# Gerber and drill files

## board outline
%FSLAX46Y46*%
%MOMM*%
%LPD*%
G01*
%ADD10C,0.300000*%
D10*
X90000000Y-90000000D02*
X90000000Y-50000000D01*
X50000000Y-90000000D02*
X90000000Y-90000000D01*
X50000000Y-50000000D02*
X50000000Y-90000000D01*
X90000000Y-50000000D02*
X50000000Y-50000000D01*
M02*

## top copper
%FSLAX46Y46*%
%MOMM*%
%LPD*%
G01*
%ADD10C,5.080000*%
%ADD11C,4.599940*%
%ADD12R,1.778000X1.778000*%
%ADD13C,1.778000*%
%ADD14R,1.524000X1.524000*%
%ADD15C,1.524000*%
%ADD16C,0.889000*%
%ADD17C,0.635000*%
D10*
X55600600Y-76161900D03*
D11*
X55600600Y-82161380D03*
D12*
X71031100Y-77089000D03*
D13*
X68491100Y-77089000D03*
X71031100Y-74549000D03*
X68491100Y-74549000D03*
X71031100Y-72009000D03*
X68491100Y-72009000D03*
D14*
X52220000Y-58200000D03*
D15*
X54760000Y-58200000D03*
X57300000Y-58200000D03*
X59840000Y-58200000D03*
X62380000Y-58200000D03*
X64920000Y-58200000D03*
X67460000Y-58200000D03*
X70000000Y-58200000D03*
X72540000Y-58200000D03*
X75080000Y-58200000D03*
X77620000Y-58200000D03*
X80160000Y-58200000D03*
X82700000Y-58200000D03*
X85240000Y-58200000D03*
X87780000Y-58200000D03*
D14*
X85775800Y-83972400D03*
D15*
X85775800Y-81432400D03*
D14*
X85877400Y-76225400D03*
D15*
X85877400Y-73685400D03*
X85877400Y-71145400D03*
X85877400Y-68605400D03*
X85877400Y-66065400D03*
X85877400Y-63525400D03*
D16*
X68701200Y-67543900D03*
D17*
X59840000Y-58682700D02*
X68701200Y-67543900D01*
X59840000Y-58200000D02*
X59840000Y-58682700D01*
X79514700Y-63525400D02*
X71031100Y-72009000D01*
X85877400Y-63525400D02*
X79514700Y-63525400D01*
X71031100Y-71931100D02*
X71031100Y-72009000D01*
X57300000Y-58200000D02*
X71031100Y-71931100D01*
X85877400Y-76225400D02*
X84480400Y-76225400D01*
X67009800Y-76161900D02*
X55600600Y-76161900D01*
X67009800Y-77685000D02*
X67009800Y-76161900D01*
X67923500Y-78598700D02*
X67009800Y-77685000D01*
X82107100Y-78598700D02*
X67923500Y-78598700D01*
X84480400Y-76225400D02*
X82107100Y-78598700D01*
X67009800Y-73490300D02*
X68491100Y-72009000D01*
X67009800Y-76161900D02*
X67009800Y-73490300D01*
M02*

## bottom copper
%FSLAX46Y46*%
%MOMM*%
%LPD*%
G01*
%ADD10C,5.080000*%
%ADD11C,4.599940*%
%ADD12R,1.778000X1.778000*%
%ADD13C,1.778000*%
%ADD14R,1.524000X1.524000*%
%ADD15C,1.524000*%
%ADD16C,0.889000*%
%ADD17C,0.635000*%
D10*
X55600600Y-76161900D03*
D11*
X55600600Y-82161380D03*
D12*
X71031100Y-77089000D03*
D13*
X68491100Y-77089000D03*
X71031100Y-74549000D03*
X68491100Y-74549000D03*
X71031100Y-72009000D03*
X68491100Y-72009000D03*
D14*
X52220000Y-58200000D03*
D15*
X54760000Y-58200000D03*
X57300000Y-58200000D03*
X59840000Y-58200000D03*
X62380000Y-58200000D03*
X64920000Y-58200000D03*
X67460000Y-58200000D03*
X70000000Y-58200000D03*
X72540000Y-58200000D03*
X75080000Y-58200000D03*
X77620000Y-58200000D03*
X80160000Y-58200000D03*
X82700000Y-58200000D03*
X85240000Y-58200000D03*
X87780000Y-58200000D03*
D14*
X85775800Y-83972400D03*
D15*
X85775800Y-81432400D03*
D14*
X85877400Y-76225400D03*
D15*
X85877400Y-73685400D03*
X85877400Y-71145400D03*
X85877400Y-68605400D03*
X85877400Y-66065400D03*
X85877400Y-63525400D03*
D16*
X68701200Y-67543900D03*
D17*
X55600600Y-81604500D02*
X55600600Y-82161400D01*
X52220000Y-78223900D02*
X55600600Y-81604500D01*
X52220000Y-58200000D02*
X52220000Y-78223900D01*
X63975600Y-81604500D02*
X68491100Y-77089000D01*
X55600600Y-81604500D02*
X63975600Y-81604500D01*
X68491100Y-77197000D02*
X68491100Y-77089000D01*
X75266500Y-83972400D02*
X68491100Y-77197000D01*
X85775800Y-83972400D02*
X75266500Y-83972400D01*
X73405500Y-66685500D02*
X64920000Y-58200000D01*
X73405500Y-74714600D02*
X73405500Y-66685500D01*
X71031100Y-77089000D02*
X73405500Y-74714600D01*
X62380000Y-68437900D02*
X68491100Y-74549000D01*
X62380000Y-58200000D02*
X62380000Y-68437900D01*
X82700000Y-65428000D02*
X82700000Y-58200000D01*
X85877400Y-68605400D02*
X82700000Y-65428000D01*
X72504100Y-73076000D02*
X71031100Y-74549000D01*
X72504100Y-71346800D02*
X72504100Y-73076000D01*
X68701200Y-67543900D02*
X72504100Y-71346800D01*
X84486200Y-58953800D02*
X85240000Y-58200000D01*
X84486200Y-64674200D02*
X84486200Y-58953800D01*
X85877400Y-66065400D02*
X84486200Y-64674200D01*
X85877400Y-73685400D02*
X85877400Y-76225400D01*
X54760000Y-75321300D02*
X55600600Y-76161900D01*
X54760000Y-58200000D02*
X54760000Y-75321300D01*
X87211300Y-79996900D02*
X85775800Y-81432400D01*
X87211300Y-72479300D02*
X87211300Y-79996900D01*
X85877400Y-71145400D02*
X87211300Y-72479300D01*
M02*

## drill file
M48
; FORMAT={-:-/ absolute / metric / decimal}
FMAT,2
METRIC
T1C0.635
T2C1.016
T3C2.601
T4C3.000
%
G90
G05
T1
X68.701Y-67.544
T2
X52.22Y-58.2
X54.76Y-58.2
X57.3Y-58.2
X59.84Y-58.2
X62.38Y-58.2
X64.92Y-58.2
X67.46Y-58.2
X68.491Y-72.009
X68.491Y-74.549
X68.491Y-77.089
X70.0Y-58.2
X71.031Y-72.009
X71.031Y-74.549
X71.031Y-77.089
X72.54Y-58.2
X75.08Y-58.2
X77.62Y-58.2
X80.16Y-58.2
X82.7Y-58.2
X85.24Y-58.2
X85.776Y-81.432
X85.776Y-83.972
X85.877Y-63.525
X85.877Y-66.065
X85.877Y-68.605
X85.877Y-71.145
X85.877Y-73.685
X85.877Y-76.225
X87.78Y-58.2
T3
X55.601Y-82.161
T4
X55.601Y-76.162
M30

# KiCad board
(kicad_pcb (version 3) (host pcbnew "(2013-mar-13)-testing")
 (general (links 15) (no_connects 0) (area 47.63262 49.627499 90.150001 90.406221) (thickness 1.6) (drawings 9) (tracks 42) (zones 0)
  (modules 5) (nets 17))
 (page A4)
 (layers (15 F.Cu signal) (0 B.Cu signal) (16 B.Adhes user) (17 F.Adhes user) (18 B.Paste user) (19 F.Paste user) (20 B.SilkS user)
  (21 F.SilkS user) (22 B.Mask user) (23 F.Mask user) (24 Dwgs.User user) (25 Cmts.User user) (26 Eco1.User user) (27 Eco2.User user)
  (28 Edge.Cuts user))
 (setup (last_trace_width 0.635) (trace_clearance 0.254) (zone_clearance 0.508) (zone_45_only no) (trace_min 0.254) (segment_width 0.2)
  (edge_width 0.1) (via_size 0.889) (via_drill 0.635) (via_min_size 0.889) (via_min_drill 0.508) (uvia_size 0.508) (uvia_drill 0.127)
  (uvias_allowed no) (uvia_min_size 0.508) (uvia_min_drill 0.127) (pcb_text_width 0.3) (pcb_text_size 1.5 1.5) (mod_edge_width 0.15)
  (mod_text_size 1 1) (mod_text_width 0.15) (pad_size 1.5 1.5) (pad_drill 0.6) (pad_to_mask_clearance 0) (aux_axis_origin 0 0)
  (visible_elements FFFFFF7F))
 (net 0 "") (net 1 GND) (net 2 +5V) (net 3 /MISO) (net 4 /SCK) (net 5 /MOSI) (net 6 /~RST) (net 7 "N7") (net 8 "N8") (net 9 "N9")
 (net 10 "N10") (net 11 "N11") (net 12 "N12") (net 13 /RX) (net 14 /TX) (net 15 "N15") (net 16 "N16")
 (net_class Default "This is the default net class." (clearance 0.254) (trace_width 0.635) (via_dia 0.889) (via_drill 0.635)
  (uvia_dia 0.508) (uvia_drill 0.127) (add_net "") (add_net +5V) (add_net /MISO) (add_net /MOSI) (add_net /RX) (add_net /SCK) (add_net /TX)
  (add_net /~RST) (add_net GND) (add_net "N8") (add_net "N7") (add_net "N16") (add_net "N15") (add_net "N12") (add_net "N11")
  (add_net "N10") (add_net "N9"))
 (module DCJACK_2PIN (layer F.Cu) (at 55.6006 76.1619 270)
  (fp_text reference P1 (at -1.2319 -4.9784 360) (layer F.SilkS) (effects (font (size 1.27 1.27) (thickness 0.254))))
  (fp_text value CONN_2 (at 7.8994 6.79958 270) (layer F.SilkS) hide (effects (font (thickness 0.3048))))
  (pad 1 thru_hole circle (at 0 0 270) (size 5.08 5.08) (drill 2.99974) (layers *.Cu *.Mask F.SilkS) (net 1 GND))
  (pad 2 thru_hole circle (at 5.99948 0 270) (size 4.59994 4.59994) (drill 2.60096) (layers *.Cu *.Mask F.SilkS) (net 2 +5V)))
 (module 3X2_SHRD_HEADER (layer F.Cu) (at 69.7611 74.549 90)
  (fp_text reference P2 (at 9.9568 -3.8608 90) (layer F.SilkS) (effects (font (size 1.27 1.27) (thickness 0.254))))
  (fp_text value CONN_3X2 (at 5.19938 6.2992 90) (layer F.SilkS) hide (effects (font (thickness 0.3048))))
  (pad 1 thru_hole rect (at -2.54 1.27 90) (size 1.778 1.778) (drill 1.016) (layers *.Cu *.Mask F.SilkS) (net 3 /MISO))
  (pad 2 thru_hole circle (at -2.54 -1.27 90) (size 1.778 1.778) (drill 1.016) (layers *.Cu *.Mask F.SilkS) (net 2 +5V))
  (pad 3 thru_hole circle (at 0 1.27 90) (size 1.778 1.778) (drill 1.016) (layers *.Cu *.Mask F.SilkS) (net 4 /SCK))
  (pad 4 thru_hole circle (at 0 -1.27 90) (size 1.778 1.778) (drill 1.016) (layers *.Cu *.Mask F.SilkS) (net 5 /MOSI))
  (pad 5 thru_hole circle (at 2.54 1.27 90) (size 1.778 1.778) (drill 1.016) (layers *.Cu *.Mask F.SilkS) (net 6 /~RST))
  (pad 6 thru_hole circle (at 2.54 -1.27 90) (size 1.778 1.778) (drill 1.016) (layers *.Cu *.Mask F.SilkS) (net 1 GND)))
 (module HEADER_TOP (layer F.Cu) (at 70 58.2)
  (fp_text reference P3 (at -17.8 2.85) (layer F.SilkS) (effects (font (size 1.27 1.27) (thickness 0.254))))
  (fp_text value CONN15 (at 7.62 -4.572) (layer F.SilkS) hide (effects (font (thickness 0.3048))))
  (pad 1 thru_hole rect (at -17.78 0) (size 1.524 1.524) (drill 1.016) (layers *.Cu *.Mask F.SilkS) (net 2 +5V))
  (pad 2 thru_hole circle (at -15.24 0) (size 1.524 1.524) (drill 1.016) (layers *.Cu *.Mask F.SilkS) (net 1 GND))
  (pad 3 thru_hole circle (at -12.7 0) (size 1.524 1.524) (drill 1.016) (layers *.Cu *.Mask F.SilkS) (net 6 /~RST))
  (pad 4 thru_hole circle (at -10.16 0) (size 1.524 1.524) (drill 1.016) (layers *.Cu *.Mask F.SilkS) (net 4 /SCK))
  (pad 5 thru_hole circle (at -7.62 0) (size 1.524 1.524) (drill 1.016) (layers *.Cu *.Mask F.SilkS) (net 5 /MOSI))
  (pad 6 thru_hole circle (at -5.08 0) (size 1.524 1.524) (drill 1.016) (layers *.Cu *.Mask F.SilkS) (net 3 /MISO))
  (pad 7 thru_hole circle (at -2.54 0) (size 1.524 1.524) (drill 1.016) (layers *.Cu *.Mask F.SilkS) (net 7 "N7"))
  (pad 8 thru_hole circle (at 0 0) (size 1.524 1.524) (drill 1.016) (layers *.Cu *.Mask F.SilkS) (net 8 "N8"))
  (pad 9 thru_hole circle (at 2.54 0) (size 1.524 1.524) (drill 1.016) (layers *.Cu *.Mask F.SilkS) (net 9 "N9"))
  (pad 10 thru_hole circle (at 5.08 0) (size 1.524 1.524) (drill 1.016) (layers *.Cu *.Mask F.SilkS) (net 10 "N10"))
  (pad 11 thru_hole circle (at 7.62 0) (size 1.524 1.524) (drill 1.016) (layers *.Cu *.Mask F.SilkS) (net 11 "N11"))
  (pad 12 thru_hole circle (at 10.16 0) (size 1.524 1.524) (drill 1.016) (layers *.Cu *.Mask F.SilkS) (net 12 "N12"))
  (pad 13 thru_hole circle (at 12.7 0) (size 1.524 1.524) (drill 1.016) (layers *.Cu *.Mask F.SilkS) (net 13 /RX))
  (pad 14 thru_hole circle (at 15.24 0) (size 1.524 1.524) (drill 1.016) (layers *.Cu *.Mask F.SilkS) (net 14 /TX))
  (pad 15 thru_hole circle (at 17.78 0) (size 1.524 1.524) (drill 1.016) (layers *.Cu *.Mask F.SilkS) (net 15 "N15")))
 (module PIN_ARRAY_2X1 (layer F.Cu) (at 85.7758 82.7024 90)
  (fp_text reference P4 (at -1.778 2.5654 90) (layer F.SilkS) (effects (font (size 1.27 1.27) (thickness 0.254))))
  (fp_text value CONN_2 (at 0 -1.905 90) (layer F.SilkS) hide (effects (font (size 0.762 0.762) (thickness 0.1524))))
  (pad 1 thru_hole rect (at -1.27 0 90) (size 1.524 1.524) (drill 1.016) (layers *.Cu *.Mask F.SilkS) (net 2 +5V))
  (pad 2 thru_hole circle (at 1.27 0 90) (size 1.524 1.524) (drill 1.016) (layers *.Cu *.Mask F.SilkS) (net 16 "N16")))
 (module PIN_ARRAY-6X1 (layer F.Cu) (at 85.8774 69.8754 90)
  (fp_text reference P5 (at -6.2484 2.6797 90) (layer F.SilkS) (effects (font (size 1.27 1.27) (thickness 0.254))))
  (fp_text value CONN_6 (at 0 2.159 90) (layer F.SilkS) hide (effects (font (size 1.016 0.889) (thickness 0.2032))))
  (pad 1 thru_hole rect (at -6.35 0 90) (size 1.524 1.524) (drill 1.016) (layers *.Cu *.Mask F.SilkS) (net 1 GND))
  (pad 2 thru_hole circle (at -3.81 0 90) (size 1.524 1.524) (drill 1.016) (layers *.Cu *.Mask F.SilkS) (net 1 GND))
  (pad 3 thru_hole circle (at -1.27 0 90) (size 1.524 1.524) (drill 1.016) (layers *.Cu *.Mask F.SilkS) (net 16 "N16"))
  (pad 4 thru_hole circle (at 1.27 0 90) (size 1.524 1.524) (drill 1.016) (layers *.Cu *.Mask F.SilkS) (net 13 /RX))
  (pad 5 thru_hole circle (at 3.81 0 90) (size 1.524 1.524) (drill 1.016) (layers *.Cu *.Mask F.SilkS) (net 14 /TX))
  (pad 6 thru_hole circle (at 6.35 0 90) (size 1.524 1.524) (drill 1.016) (layers *.Cu *.Mask F.SilkS) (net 6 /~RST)))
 (gr_line (start 90 90) (end 90 50) (angle 90) (layer Edge.Cuts) (width 0.3))
 (gr_line (start 50 90) (end 90 90) (angle 90) (layer Edge.Cuts) (width 0.3))
 (gr_line (start 50 50) (end 50 90) (angle 90) (layer Edge.Cuts) (width 0.3))
 (gr_line (start 90 50) (end 50 50) (angle 90) (layer Edge.Cuts) (width 0.3))
 (segment (start 55.6006 81.6045) (end 55.6006 82.1614) (width 0.635) (layer B.Cu) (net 2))
 (segment (start 52.22 78.2239) (end 55.6006 81.6045) (width 0.635) (layer B.Cu) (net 2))
 (segment (start 52.22 58.2) (end 52.22 78.2239) (width 0.635) (layer B.Cu) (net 2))
 (segment (start 63.9756 81.6045) (end 68.4911 77.089) (width 0.635) (layer B.Cu) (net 2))
 (segment (start 55.6006 81.6045) (end 63.9756 81.6045) (width 0.635) (layer B.Cu) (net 2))
 (segment (start 68.4911 77.197) (end 68.4911 77.089) (width 0.635) (layer B.Cu) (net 2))
 (segment (start 75.2665 83.9724) (end 68.4911 77.197) (width 0.635) (layer B.Cu) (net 2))
 (segment (start 85.7758 83.9724) (end 75.2665 83.9724) (width 0.635) (layer B.Cu) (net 2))
 (segment (start 73.4055 66.6855) (end 64.92 58.2) (width 0.635) (layer B.Cu) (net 3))
 (segment (start 73.4055 74.7146) (end 73.4055 66.6855) (width 0.635) (layer B.Cu) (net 3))
 (segment (start 71.0311 77.089) (end 73.4055 74.7146) (width 0.635) (layer B.Cu) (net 3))
 (segment (start 62.38 68.4379) (end 68.4911 74.549) (width 0.635) (layer B.Cu) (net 5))
 (segment (start 62.38 58.2) (end 62.38 68.4379) (width 0.635) (layer B.Cu) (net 5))
 (segment (start 82.7 65.428) (end 82.7 58.2) (width 0.635) (layer B.Cu) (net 13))
 (segment (start 85.8774 68.6054) (end 82.7 65.428) (width 0.635) (layer B.Cu) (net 13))
 (via (at 68.7012 67.5439) (size 0.889) (layers F.Cu B.Cu) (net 4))
 (segment (start 72.5041 73.076) (end 71.0311 74.549) (width 0.635) (layer B.Cu) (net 4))
 (segment (start 72.5041 71.3468) (end 72.5041 73.076) (width 0.635) (layer B.Cu) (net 4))
 (segment (start 68.7012 67.5439) (end 72.5041 71.3468) (width 0.635) (layer B.Cu) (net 4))
 (segment (start 59.84 58.6827) (end 68.7012 67.5439) (width 0.635) (layer F.Cu) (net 4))
 (segment (start 59.84 58.2) (end 59.84 58.6827) (width 0.635) (layer F.Cu) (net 4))
 (segment (start 84.4862 58.9538) (end 85.24 58.2) (width 0.635) (layer B.Cu) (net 14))
 (segment (start 84.4862 64.6742) (end 84.4862 58.9538) (width 0.635) (layer B.Cu) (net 14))
 (segment (start 85.8774 66.0654) (end 84.4862 64.6742) (width 0.635) (layer B.Cu) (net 14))
 (segment (start 79.5147 63.5254) (end 71.0311 72.009) (width 0.635) (layer F.Cu) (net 6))
 (segment (start 85.8774 63.5254) (end 79.5147 63.5254) (width 0.635) (layer F.Cu) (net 6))
 (segment (start 71.0311 71.9311) (end 71.0311 72.009) (width 0.635) (layer F.Cu) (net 6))
 (segment (start 57.3 58.2) (end 71.0311 71.9311) (width 0.635) (layer F.Cu) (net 6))
 (segment (start 85.8774 73.6854) (end 85.8774 76.2254) (width 0.635) (layer B.Cu) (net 1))
 (segment (start 54.76 75.3213) (end 55.6006 76.1619) (width 0.635) (layer B.Cu) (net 1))
 (segment (start 54.76 58.2) (end 54.76 75.3213) (width 0.635) (layer B.Cu) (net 1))
 (segment (start 85.8774 76.2254) (end 84.4804 76.2254) (width 0.635) (layer F.Cu) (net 1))
 (segment (start 67.0098 76.1619) (end 55.6006 76.1619) (width 0.635) (layer F.Cu) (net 1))
 (segment (start 67.0098 77.685) (end 67.0098 76.1619) (width 0.635) (layer F.Cu) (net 1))
 (segment (start 67.9235 78.5987) (end 67.0098 77.685) (width 0.635) (layer F.Cu) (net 1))
 (segment (start 82.1071 78.5987) (end 67.9235 78.5987) (width 0.635) (layer F.Cu) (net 1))
 (segment (start 84.4804 76.2254) (end 82.1071 78.5987) (width 0.635) (layer F.Cu) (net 1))
 (segment (start 67.0098 73.4903) (end 68.4911 72.009) (width 0.635) (layer F.Cu) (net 1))
 (segment (start 67.0098 76.1619) (end 67.0098 73.4903) (width 0.635) (layer F.Cu) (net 1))
 (segment (start 87.2113 79.9969) (end 85.7758 81.4324) (width 0.635) (layer B.Cu) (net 16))
 (segment (start 87.2113 72.4793) (end 87.2113 79.9969) (width 0.635) (layer B.Cu) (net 16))
 (segment (start 85.8774 71.1454) (end 87.2113 72.4793) (width 0.635) (layer B.Cu) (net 16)))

